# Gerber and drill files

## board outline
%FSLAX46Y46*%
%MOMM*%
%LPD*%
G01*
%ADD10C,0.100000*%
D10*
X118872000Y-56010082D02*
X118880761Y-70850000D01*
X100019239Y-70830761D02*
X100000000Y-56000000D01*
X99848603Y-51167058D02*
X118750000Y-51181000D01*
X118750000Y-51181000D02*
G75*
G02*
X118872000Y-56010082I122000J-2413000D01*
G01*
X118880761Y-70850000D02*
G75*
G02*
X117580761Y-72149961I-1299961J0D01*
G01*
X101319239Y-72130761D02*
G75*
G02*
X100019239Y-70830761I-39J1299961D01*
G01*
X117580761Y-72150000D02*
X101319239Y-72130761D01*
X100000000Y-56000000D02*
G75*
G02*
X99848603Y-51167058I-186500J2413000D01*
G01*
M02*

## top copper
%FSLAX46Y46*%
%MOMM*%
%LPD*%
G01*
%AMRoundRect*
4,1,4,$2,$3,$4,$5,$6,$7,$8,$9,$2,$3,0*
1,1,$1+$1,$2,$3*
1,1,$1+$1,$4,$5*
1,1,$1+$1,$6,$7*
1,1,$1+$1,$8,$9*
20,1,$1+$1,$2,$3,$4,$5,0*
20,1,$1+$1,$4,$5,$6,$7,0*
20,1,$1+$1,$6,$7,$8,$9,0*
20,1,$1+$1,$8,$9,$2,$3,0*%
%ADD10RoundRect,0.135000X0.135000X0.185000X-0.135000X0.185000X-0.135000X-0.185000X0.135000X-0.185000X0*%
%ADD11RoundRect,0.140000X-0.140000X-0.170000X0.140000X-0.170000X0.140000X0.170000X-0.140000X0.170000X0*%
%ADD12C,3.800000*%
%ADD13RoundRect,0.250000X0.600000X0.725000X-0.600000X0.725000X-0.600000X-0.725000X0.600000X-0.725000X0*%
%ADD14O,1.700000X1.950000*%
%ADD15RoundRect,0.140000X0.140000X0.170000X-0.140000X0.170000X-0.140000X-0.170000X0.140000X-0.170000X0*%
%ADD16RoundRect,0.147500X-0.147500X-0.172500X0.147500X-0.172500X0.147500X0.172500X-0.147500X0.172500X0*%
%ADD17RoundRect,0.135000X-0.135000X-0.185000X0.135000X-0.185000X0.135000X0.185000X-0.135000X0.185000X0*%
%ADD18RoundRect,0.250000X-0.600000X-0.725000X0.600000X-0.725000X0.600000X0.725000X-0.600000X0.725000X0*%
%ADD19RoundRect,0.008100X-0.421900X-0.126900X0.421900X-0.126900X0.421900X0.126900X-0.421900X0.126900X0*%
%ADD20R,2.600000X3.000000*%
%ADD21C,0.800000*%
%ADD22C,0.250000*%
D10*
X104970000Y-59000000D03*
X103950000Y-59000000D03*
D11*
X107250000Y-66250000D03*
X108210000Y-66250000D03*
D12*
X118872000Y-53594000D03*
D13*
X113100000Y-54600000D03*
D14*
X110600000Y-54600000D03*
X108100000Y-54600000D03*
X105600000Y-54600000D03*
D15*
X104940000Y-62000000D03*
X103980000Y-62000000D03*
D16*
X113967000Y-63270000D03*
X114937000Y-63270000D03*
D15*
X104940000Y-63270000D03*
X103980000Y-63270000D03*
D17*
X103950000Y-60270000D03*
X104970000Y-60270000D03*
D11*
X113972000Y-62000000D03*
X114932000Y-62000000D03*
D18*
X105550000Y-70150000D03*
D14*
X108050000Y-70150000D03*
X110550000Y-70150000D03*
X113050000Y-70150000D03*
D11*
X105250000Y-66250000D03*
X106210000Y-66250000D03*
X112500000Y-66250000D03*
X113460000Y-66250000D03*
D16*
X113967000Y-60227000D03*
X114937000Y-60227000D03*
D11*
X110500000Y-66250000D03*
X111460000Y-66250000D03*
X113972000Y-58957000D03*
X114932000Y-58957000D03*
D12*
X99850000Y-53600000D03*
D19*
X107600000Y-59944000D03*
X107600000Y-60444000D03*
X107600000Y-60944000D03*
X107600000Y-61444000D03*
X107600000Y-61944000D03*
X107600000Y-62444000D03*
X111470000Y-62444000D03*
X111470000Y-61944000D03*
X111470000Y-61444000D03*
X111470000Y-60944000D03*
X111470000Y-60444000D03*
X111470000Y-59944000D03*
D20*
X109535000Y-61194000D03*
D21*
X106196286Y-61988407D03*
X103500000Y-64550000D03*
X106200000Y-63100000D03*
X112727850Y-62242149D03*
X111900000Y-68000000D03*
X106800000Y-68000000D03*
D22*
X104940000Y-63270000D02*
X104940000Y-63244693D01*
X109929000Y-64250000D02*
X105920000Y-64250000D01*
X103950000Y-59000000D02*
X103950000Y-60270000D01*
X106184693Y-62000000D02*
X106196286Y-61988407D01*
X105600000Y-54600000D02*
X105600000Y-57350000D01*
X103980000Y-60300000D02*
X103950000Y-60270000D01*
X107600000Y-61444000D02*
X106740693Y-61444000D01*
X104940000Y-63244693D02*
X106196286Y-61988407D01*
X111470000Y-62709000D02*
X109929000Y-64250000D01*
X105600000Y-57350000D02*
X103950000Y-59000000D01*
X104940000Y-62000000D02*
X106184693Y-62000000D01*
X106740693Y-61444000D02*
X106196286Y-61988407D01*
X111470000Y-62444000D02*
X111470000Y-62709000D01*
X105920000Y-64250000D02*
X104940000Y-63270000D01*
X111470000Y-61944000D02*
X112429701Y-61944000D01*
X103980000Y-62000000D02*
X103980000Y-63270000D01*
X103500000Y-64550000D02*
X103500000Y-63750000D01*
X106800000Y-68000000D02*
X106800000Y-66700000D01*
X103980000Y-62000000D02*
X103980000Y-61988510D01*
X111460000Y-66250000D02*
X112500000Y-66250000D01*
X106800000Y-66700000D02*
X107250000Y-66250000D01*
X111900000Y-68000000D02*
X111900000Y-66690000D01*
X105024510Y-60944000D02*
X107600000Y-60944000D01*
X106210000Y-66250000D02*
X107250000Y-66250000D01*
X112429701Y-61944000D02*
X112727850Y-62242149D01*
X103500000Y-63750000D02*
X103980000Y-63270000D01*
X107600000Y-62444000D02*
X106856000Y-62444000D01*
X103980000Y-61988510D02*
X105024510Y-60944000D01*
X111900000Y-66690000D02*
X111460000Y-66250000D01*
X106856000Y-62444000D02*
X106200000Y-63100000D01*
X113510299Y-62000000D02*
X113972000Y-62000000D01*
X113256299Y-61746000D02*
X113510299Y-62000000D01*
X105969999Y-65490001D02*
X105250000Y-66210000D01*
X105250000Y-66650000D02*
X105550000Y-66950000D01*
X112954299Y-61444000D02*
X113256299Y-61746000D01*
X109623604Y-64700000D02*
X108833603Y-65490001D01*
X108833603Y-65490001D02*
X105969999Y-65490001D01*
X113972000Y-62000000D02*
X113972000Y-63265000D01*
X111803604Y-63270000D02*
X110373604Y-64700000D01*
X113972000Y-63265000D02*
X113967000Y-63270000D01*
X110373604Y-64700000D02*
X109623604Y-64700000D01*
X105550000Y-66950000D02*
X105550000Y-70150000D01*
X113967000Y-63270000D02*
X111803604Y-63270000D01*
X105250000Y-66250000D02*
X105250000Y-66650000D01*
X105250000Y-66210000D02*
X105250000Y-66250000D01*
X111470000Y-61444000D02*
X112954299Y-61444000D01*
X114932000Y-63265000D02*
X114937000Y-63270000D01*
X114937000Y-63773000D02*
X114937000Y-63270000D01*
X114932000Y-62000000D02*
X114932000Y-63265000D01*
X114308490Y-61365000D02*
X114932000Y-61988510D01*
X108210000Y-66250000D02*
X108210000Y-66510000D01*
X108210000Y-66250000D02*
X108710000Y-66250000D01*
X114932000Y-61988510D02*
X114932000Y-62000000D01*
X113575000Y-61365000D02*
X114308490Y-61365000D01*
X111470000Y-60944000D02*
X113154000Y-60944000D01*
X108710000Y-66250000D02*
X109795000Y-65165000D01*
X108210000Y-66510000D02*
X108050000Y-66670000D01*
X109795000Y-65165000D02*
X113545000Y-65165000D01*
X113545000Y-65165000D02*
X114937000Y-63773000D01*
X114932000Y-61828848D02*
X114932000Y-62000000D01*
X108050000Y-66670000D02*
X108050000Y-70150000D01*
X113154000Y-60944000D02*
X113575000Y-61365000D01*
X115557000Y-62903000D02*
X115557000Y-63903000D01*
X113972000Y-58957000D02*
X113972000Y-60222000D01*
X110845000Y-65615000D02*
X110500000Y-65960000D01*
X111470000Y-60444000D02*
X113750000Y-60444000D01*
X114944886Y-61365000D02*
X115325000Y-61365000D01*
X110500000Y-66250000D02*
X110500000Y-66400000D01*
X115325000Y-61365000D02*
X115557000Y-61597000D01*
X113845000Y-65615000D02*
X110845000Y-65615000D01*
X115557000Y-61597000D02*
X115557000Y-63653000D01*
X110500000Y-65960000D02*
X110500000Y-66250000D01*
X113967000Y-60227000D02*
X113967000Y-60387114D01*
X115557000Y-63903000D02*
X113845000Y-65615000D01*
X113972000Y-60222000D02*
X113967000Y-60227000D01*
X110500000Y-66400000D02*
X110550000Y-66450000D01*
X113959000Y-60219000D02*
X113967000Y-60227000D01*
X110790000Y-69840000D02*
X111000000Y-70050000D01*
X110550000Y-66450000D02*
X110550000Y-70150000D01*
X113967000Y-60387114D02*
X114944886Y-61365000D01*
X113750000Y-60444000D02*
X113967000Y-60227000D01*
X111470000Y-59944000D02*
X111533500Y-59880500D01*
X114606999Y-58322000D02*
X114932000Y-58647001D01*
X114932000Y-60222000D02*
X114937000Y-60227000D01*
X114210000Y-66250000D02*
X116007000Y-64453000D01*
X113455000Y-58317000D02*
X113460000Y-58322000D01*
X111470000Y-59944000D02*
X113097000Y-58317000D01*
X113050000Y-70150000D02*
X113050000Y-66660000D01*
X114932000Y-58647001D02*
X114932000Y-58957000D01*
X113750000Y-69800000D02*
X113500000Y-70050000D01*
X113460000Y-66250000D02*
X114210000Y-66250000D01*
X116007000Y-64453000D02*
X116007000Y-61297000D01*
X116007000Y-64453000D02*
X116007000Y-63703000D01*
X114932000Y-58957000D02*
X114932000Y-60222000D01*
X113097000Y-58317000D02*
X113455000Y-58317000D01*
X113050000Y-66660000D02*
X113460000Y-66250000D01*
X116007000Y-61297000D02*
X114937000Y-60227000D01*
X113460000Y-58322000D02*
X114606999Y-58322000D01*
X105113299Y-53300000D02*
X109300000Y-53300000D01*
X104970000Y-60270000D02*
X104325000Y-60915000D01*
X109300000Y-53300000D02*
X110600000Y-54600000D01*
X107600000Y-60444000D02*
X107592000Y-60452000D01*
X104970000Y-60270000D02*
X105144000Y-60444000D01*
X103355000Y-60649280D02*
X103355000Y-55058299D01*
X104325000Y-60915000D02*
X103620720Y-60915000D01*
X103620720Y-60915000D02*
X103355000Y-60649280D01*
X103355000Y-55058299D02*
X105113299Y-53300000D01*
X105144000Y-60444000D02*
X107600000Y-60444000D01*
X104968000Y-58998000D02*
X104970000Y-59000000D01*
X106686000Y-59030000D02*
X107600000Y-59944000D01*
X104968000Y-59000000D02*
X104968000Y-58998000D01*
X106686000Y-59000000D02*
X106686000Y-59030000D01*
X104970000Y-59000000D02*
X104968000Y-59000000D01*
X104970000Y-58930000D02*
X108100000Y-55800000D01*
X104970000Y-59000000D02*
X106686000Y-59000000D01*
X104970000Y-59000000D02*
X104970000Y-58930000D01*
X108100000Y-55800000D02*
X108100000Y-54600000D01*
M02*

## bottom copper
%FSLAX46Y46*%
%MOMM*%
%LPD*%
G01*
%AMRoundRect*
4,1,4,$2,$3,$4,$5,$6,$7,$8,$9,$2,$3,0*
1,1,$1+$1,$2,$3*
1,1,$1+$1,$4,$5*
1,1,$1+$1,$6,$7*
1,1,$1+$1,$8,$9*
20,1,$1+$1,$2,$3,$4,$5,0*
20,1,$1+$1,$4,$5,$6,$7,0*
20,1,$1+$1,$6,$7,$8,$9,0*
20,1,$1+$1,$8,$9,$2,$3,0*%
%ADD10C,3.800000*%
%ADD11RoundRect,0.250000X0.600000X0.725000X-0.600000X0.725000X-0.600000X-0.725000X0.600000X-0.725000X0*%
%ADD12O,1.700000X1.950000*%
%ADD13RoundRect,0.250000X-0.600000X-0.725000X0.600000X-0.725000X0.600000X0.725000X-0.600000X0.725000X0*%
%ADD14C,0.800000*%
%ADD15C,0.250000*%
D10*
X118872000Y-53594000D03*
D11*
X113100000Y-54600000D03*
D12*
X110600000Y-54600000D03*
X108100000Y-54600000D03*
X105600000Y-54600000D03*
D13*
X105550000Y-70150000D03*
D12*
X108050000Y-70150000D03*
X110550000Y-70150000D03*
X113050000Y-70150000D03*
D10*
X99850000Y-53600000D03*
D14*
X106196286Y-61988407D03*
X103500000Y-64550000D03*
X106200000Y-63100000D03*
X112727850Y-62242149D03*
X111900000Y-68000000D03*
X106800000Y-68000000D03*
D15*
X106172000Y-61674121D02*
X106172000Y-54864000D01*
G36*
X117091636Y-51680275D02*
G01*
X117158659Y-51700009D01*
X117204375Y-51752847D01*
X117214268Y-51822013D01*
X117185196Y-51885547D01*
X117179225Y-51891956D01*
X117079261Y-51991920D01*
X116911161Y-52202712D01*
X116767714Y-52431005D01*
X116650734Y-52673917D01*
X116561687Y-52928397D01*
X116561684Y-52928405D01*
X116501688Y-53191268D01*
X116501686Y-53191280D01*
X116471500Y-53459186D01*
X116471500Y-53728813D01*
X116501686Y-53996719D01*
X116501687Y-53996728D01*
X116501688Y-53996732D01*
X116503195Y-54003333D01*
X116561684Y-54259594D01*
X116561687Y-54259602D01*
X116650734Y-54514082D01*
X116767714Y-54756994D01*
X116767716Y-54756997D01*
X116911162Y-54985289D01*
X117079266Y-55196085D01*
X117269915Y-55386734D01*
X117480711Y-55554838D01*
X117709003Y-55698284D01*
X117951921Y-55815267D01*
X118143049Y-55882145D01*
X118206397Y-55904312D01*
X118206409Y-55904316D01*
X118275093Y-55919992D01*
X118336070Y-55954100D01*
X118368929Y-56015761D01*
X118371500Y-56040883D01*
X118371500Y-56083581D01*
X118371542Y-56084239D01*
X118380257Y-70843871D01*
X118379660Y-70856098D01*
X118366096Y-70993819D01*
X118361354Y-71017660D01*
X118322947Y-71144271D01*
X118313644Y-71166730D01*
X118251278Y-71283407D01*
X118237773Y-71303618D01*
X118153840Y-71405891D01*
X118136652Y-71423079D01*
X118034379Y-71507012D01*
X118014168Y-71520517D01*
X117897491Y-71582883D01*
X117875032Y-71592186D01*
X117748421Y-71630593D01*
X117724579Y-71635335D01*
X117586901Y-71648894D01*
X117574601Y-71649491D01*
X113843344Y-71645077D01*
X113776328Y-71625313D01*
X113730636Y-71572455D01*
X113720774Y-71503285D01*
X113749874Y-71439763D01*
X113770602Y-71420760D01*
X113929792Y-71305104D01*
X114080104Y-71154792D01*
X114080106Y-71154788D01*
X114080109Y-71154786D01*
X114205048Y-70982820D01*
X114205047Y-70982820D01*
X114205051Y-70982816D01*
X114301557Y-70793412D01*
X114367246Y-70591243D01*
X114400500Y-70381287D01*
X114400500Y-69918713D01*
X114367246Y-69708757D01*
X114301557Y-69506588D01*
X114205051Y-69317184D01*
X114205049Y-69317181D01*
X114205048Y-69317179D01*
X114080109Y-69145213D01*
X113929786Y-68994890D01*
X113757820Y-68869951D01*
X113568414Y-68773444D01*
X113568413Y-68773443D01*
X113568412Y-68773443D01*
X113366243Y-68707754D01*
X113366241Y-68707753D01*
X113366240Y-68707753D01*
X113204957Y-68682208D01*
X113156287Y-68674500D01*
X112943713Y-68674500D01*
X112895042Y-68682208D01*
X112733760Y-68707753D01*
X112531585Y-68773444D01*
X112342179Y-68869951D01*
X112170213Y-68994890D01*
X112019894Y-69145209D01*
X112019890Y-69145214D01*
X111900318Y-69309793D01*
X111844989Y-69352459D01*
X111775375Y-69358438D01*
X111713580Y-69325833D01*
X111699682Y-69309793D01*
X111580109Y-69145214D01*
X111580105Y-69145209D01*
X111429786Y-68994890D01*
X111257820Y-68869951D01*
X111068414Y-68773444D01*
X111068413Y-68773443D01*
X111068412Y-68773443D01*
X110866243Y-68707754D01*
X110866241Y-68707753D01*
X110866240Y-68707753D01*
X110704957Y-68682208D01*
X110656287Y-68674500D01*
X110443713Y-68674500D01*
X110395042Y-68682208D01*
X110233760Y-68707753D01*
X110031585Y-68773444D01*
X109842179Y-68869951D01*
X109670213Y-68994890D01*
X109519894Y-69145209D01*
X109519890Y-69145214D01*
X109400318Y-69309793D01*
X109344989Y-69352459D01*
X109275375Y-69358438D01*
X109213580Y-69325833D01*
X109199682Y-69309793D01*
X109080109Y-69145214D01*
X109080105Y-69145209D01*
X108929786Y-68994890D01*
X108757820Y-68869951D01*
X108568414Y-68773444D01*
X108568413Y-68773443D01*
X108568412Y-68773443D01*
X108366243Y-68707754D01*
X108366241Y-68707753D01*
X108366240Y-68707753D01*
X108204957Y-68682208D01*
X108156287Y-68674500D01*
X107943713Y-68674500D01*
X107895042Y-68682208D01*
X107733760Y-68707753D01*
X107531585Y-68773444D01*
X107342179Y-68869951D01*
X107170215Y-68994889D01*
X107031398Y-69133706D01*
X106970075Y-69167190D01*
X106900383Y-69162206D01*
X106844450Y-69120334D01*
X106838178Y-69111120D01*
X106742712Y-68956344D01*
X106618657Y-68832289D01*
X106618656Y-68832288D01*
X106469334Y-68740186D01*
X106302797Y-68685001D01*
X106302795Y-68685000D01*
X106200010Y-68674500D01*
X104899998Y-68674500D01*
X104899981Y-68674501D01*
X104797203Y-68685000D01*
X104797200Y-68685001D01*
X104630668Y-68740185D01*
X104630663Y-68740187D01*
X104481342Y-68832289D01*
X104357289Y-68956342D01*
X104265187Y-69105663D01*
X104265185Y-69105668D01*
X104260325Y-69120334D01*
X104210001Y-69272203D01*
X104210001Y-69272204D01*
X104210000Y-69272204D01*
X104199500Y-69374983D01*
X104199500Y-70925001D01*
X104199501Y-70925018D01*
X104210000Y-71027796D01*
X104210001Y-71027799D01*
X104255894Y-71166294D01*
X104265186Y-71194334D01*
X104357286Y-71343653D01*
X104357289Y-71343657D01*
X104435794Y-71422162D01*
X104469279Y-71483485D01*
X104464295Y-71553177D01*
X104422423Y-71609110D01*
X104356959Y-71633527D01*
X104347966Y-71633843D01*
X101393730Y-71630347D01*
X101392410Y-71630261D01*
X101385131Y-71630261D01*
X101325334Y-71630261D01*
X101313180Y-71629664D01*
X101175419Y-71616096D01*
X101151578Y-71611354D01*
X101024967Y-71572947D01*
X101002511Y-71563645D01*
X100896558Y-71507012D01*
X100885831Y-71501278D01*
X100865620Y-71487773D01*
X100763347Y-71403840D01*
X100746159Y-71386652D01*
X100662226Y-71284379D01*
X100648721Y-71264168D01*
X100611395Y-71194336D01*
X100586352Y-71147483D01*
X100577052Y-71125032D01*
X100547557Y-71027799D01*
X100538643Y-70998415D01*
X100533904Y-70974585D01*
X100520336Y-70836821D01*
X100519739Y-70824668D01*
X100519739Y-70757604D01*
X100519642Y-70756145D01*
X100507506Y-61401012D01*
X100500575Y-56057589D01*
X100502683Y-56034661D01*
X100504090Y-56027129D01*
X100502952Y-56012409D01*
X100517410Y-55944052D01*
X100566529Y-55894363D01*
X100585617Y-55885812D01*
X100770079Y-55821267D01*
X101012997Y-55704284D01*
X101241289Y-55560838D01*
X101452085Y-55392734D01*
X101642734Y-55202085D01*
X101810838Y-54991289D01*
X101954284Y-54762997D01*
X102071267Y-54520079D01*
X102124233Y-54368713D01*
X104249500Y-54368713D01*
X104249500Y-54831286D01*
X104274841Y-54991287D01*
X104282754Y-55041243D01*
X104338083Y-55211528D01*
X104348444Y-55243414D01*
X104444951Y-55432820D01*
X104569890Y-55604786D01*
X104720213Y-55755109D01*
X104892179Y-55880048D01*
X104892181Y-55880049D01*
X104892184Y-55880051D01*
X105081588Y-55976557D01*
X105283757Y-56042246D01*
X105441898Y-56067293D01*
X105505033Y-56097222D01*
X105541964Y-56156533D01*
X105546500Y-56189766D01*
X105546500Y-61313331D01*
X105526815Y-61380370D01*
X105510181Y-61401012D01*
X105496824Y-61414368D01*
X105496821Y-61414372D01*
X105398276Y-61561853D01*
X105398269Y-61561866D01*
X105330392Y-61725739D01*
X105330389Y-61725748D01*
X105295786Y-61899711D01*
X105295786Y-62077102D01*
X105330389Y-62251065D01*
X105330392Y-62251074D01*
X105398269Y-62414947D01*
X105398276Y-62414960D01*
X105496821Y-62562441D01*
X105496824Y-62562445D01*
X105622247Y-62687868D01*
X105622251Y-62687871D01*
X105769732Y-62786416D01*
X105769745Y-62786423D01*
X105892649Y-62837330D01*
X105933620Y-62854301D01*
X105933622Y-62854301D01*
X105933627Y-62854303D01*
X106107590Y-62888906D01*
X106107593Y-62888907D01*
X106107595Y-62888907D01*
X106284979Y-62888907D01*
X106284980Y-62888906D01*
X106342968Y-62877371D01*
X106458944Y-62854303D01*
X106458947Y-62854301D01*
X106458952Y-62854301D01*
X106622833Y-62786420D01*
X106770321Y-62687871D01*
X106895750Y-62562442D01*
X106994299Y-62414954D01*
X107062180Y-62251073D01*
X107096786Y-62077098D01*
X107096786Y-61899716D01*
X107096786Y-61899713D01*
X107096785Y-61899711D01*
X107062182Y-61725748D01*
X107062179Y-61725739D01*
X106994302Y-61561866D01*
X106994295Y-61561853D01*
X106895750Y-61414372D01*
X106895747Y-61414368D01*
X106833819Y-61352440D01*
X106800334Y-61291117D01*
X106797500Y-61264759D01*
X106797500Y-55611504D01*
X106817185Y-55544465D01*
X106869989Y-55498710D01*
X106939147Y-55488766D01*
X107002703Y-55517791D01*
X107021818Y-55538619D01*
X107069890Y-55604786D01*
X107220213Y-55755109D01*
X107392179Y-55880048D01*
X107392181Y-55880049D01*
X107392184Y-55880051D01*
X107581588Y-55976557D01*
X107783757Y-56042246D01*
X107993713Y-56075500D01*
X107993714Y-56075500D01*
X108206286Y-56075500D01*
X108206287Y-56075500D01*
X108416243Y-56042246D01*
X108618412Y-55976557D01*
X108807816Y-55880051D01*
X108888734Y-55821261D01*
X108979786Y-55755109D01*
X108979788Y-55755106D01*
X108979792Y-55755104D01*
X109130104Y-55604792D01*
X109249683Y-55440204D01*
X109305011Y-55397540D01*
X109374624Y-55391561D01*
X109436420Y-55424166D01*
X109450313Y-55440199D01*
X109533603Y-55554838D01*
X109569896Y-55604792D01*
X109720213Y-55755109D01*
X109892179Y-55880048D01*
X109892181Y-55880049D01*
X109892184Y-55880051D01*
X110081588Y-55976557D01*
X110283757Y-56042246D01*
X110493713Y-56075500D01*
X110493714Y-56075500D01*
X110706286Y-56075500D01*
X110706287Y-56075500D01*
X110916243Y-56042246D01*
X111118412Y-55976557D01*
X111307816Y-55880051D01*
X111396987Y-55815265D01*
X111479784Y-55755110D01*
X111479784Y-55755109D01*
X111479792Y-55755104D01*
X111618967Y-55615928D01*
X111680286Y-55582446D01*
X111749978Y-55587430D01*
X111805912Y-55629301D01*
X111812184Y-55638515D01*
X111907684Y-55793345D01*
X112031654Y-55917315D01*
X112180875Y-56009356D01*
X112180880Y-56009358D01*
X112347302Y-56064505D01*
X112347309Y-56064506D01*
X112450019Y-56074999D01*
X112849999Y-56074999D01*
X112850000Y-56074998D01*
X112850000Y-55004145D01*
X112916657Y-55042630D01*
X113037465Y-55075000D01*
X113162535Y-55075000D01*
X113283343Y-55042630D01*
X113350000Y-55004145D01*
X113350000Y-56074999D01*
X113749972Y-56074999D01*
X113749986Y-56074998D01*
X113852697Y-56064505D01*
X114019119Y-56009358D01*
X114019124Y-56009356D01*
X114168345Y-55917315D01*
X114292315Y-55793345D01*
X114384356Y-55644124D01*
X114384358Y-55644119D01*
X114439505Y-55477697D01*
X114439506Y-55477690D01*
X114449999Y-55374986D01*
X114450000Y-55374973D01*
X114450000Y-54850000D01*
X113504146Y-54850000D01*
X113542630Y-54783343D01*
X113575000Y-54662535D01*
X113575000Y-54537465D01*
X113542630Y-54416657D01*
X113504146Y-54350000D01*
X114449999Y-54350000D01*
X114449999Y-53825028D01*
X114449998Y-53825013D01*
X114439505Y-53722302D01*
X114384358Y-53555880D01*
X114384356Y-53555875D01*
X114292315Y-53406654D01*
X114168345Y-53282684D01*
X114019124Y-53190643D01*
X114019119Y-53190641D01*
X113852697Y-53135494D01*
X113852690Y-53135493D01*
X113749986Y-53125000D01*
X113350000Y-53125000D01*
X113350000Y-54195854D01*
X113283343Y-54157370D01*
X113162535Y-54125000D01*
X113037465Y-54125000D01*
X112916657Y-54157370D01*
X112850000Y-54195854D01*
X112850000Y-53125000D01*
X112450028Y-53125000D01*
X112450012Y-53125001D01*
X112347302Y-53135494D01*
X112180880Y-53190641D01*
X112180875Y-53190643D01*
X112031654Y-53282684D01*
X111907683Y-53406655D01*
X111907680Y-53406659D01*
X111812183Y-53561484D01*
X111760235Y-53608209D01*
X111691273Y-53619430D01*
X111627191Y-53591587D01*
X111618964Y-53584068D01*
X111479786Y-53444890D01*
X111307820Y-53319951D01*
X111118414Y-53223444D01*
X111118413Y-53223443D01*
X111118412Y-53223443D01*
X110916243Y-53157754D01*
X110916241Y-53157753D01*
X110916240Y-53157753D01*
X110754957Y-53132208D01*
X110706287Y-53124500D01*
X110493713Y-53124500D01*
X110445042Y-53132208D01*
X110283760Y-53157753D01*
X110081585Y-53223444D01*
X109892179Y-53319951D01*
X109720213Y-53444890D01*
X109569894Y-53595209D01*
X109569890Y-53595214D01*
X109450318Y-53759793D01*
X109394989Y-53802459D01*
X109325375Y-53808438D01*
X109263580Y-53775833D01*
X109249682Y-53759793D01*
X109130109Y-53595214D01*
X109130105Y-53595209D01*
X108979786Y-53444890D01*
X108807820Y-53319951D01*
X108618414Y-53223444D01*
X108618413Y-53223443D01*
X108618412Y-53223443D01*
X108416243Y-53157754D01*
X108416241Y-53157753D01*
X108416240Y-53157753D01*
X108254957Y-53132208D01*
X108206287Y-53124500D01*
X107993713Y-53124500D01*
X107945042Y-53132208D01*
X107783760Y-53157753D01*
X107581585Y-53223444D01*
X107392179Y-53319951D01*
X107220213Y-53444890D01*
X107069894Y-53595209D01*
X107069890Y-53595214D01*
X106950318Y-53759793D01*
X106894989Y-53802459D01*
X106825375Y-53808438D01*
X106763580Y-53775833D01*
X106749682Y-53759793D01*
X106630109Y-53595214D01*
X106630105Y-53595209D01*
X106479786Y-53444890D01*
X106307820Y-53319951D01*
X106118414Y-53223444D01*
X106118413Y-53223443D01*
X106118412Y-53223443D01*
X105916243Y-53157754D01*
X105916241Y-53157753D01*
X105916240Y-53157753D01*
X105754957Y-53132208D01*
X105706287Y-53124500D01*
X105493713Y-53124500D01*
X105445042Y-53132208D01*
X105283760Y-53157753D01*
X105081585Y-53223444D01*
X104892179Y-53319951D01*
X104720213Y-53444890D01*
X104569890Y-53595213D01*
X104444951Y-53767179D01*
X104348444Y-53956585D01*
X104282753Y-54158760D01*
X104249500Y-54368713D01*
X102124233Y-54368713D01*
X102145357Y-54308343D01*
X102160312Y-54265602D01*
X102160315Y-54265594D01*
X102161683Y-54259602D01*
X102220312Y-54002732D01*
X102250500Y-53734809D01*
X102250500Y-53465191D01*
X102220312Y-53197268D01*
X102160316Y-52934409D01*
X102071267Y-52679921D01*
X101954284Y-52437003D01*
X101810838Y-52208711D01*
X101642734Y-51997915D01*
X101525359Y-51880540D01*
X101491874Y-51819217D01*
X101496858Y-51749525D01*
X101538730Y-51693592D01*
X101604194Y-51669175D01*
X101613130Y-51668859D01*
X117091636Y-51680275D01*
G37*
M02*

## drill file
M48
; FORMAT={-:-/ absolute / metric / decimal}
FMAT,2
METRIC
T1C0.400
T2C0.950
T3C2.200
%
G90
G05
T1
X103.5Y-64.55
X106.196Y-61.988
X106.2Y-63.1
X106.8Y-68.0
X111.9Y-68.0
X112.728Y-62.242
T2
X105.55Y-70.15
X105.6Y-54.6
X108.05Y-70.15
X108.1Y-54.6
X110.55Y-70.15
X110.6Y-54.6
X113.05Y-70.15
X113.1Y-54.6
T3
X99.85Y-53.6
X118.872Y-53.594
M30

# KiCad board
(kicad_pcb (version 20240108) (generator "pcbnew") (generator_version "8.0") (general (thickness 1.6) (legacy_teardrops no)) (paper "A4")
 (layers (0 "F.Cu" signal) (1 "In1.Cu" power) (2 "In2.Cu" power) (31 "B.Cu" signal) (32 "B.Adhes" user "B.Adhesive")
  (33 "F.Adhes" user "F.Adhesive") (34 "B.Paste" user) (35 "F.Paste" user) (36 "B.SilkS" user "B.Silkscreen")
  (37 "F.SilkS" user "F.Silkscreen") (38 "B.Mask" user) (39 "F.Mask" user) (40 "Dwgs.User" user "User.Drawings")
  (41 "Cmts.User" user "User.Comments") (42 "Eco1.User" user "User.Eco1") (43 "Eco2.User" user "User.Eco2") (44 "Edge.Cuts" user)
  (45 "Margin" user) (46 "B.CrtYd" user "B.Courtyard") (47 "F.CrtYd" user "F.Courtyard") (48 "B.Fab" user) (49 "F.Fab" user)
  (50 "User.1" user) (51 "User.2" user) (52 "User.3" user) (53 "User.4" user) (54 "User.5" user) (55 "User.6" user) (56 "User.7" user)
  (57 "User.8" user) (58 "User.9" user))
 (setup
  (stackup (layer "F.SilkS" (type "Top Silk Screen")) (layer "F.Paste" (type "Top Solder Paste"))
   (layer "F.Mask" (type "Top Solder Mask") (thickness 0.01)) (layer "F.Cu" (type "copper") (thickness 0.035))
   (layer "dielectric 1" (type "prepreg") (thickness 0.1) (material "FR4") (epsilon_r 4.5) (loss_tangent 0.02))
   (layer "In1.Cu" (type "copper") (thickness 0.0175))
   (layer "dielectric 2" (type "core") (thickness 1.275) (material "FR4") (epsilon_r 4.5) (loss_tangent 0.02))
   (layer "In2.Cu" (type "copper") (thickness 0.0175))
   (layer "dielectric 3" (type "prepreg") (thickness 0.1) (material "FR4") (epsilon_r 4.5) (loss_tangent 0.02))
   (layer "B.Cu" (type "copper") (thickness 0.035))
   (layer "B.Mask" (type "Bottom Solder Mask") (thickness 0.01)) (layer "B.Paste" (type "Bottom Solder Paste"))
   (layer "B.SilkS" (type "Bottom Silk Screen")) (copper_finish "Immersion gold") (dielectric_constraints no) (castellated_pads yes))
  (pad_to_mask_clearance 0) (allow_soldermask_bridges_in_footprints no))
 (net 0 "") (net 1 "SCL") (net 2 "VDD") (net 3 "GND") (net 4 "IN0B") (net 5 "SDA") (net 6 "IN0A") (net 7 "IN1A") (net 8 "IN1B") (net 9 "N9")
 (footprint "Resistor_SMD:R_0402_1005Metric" (layer "F.Cu") (at 104.46 59 180)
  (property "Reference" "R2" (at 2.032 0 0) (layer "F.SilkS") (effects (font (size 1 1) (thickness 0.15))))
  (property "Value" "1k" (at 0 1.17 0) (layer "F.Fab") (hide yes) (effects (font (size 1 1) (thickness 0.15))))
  (pad "1" smd roundrect (at -0.51 0 180) (size 0.54 0.64) (layers "F.Cu" "F.Paste" "F.Mask") (roundrect_rratio 0.25) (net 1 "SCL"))
  (pad "2" smd roundrect (at 0.51 0 180) (size 0.54 0.64) (layers "F.Cu" "F.Paste" "F.Mask") (roundrect_rratio 0.25) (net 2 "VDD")))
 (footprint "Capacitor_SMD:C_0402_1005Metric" (layer "F.Cu") (at 107.73 66.25)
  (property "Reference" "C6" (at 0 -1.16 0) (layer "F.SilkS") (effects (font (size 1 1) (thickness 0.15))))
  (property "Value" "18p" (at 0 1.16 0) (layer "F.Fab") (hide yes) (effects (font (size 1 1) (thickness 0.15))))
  (pad "1" smd roundrect (at -0.48 0) (size 0.56 0.62) (layers "F.Cu" "F.Paste" "F.Mask") (roundrect_rratio 0.25) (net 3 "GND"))
  (pad "2" smd roundrect (at 0.48 0) (size 0.56 0.62) (layers "F.Cu" "F.Paste" "F.Mask") (roundrect_rratio 0.25) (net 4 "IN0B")))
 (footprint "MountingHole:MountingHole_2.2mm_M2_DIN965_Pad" (layer "F.Cu") (at 118.872 53.594)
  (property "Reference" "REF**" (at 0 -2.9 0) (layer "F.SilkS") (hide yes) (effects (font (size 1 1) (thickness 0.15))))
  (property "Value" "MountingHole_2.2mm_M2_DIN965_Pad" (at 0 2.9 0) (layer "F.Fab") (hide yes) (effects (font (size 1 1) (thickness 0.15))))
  (pad "1" thru_hole circle (at 0 0) (size 3.8 3.8) (drill 2.2) (layers "*.Cu" "*.Mask") (remove_unused_layers no)))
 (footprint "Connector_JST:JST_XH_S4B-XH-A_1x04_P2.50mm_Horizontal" (layer "F.Cu") (at 113.1 54.6 180)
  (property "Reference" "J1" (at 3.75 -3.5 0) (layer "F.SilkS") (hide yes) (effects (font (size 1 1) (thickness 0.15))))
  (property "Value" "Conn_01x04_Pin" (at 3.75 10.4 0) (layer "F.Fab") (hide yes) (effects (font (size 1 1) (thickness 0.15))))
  (pad "1" thru_hole roundrect (at 0 0 180) (size 1.7 1.95) (drill 0.95) (layers "*.Cu" "*.Mask") (remove_unused_layers no)
   (roundrect_rratio 0.147059) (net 3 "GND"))
  (pad "2" thru_hole oval (at 2.5 0 180) (size 1.7 1.95) (drill 0.95) (layers "*.Cu" "*.Mask") (remove_unused_layers no) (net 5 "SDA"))
  (pad "3" thru_hole oval (at 5 0 180) (size 1.7 1.95) (drill 0.95) (layers "*.Cu" "*.Mask") (remove_unused_layers no) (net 1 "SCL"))
  (pad "4" thru_hole oval (at 7.5 0 180) (size 1.7 1.95) (drill 0.95) (layers "*.Cu" "*.Mask") (remove_unused_layers no) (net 2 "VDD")))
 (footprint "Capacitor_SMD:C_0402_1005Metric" (layer "F.Cu") (at 104.46 62 180)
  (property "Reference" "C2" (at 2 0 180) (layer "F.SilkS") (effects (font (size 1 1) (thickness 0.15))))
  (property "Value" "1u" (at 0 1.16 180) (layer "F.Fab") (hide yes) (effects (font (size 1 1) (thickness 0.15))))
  (pad "1" smd roundrect (at -0.48 0 180) (size 0.56 0.62) (layers "F.Cu" "F.Paste" "F.Mask") (roundrect_rratio 0.25) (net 2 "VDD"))
  (pad "2" smd roundrect (at 0.48 0 180) (size 0.56 0.62) (layers "F.Cu" "F.Paste" "F.Mask") (roundrect_rratio 0.25) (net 3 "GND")))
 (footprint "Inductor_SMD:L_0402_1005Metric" (layer "F.Cu") (at 114.452 63.27)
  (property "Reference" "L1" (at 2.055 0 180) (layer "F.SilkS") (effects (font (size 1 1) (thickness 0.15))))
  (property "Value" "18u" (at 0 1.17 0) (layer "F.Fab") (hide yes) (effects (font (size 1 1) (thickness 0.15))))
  (pad "1" smd roundrect (at -0.485 0) (size 0.59 0.64) (layers "F.Cu" "F.Paste" "F.Mask") (roundrect_rratio 0.25) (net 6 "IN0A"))
  (pad "2" smd roundrect (at 0.485 0) (size 0.59 0.64) (layers "F.Cu" "F.Paste" "F.Mask") (roundrect_rratio 0.25) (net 4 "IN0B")))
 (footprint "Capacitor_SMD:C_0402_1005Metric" (layer "F.Cu") (at 104.46 63.27 180)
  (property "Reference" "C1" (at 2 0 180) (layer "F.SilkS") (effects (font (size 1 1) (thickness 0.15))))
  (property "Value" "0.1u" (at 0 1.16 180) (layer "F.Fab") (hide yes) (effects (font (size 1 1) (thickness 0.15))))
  (pad "1" smd roundrect (at -0.48 0 180) (size 0.56 0.62) (layers "F.Cu" "F.Paste" "F.Mask") (roundrect_rratio 0.25) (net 2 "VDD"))
  (pad "2" smd roundrect (at 0.48 0 180) (size 0.56 0.62) (layers "F.Cu" "F.Paste" "F.Mask") (roundrect_rratio 0.25) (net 3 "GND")))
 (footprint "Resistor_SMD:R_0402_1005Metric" (layer "F.Cu") (at 104.46 60.27)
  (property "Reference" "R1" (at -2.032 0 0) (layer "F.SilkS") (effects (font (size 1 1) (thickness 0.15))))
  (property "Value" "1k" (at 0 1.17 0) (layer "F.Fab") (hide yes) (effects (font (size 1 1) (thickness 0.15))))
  (pad "1" smd roundrect (at -0.51 0) (size 0.54 0.64) (layers "F.Cu" "F.Paste" "F.Mask") (roundrect_rratio 0.25) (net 2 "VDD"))
  (pad "2" smd roundrect (at 0.51 0) (size 0.54 0.64) (layers "F.Cu" "F.Paste" "F.Mask") (roundrect_rratio 0.25) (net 5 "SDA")))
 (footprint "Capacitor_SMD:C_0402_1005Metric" (layer "F.Cu") (at 114.452 62)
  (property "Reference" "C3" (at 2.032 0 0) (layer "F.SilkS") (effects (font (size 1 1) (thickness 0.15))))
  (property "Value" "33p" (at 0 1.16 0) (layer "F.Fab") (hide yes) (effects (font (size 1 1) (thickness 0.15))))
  (pad "1" smd roundrect (at -0.48 0) (size 0.56 0.62) (layers "F.Cu" "F.Paste" "F.Mask") (roundrect_rratio 0.25) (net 6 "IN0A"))
  (pad "2" smd roundrect (at 0.48 0) (size 0.56 0.62) (layers "F.Cu" "F.Paste" "F.Mask") (roundrect_rratio 0.25) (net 4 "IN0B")))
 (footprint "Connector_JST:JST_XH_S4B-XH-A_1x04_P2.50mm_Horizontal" (layer "F.Cu") (at 105.55 70.15)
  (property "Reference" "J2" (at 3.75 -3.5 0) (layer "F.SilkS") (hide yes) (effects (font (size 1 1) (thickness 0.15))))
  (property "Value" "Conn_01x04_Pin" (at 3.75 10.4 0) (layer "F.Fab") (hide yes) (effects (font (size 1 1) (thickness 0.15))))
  (pad "1" thru_hole roundrect (at 0 0) (size 1.7 1.95) (drill 0.95) (layers "*.Cu" "*.Mask") (remove_unused_layers no)
   (roundrect_rratio 0.147059) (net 6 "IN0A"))
  (pad "2" thru_hole oval (at 2.5 0) (size 1.7 1.95) (drill 0.95) (layers "*.Cu" "*.Mask") (remove_unused_layers no) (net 4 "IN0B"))
  (pad "3" thru_hole oval (at 5 0) (size 1.7 1.95) (drill 0.95) (layers "*.Cu" "*.Mask") (remove_unused_layers no) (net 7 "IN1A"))
  (pad "4" thru_hole oval (at 7.5 0) (size 1.7 1.95) (drill 0.95) (layers "*.Cu" "*.Mask") (remove_unused_layers no) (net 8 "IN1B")))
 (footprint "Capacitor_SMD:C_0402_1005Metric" (layer "F.Cu") (at 105.73 66.25)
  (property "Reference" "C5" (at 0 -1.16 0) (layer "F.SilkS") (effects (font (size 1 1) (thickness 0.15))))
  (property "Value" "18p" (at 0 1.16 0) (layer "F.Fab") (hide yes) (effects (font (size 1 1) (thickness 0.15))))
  (pad "1" smd roundrect (at -0.48 0) (size 0.56 0.62) (layers "F.Cu" "F.Paste" "F.Mask") (roundrect_rratio 0.25) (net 6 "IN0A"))
  (pad "2" smd roundrect (at 0.48 0) (size 0.56 0.62) (layers "F.Cu" "F.Paste" "F.Mask") (roundrect_rratio 0.25) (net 3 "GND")))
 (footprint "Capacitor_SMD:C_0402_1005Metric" (layer "F.Cu") (at 112.98 66.25)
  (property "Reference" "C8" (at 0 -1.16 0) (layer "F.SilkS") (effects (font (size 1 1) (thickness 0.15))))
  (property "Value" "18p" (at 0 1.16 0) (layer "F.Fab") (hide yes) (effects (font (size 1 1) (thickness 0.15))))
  (pad "1" smd roundrect (at -0.48 0) (size 0.56 0.62) (layers "F.Cu" "F.Paste" "F.Mask") (roundrect_rratio 0.25) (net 3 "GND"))
  (pad "2" smd roundrect (at 0.48 0) (size 0.56 0.62) (layers "F.Cu" "F.Paste" "F.Mask") (roundrect_rratio 0.25) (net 8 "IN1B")))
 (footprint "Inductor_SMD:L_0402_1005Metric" (layer "F.Cu") (at 114.452 60.227)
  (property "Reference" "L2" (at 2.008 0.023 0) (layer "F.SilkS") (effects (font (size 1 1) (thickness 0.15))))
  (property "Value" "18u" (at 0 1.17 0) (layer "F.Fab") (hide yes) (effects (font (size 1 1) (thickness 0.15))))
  (pad "1" smd roundrect (at -0.485 0) (size 0.59 0.64) (layers "F.Cu" "F.Paste" "F.Mask") (roundrect_rratio 0.25) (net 7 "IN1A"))
  (pad "2" smd roundrect (at 0.485 0) (size 0.59 0.64) (layers "F.Cu" "F.Paste" "F.Mask") (roundrect_rratio 0.25) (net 8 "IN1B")))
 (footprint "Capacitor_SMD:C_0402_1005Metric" (layer "F.Cu") (at 110.98 66.25)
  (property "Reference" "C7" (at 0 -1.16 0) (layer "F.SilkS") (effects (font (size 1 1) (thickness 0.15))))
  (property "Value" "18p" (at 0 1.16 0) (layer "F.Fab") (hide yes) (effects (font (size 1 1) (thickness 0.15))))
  (pad "1" smd roundrect (at -0.48 0) (size 0.56 0.62) (layers "F.Cu" "F.Paste" "F.Mask") (roundrect_rratio 0.25) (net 7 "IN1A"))
  (pad "2" smd roundrect (at 0.48 0) (size 0.56 0.62) (layers "F.Cu" "F.Paste" "F.Mask") (roundrect_rratio 0.25) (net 3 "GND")))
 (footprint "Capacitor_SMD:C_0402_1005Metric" (layer "F.Cu") (at 114.452 58.957)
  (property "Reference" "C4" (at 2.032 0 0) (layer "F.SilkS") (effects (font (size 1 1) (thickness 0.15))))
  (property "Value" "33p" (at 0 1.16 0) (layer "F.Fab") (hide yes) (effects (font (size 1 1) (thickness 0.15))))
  (pad "1" smd roundrect (at -0.48 0) (size 0.56 0.62) (layers "F.Cu" "F.Paste" "F.Mask") (roundrect_rratio 0.25) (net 7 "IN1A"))
  (pad "2" smd roundrect (at 0.48 0) (size 0.56 0.62) (layers "F.Cu" "F.Paste" "F.Mask") (roundrect_rratio 0.25) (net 8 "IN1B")))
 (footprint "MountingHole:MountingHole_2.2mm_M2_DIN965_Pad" (layer "F.Cu") (at 99.85 53.6)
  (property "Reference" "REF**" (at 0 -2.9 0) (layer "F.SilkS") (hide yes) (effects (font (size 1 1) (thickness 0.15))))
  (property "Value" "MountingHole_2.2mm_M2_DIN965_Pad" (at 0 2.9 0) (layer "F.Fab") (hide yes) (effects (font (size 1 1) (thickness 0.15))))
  (pad "1" thru_hole circle (at 0 0) (size 3.8 3.8) (drill 2.2) (layers "*.Cu" "*.Mask") (remove_unused_layers no)))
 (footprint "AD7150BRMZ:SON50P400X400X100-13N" (layer "F.Cu") (at 109.535 61.194)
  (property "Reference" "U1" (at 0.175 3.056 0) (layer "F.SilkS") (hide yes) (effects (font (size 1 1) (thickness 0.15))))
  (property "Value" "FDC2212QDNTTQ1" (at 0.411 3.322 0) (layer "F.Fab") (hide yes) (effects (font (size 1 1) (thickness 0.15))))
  (pad "1" smd roundrect (at -1.935 -1.25) (size 0.86 0.27) (layers "F.Cu" "F.Paste" "F.Mask") (roundrect_rratio 0.03) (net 1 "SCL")
   (solder_mask_margin 0.102))
  (pad "2" smd roundrect (at -1.935 -0.75) (size 0.86 0.27) (layers "F.Cu" "F.Paste" "F.Mask") (roundrect_rratio 0.03) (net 5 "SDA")
   (solder_mask_margin 0.102))
  (pad "3" smd roundrect (at -1.935 -0.25) (size 0.86 0.27) (layers "F.Cu" "F.Paste" "F.Mask") (roundrect_rratio 0.03) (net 3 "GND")
   (solder_mask_margin 0.102))
  (pad "4" smd roundrect (at -1.935 0.25) (size 0.86 0.27) (layers "F.Cu" "F.Paste" "F.Mask") (roundrect_rratio 0.03) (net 2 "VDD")
   (solder_mask_margin 0.102))
  (pad "5" smd roundrect (at -1.935 0.75) (size 0.86 0.27) (layers "F.Cu" "F.Paste" "F.Mask") (roundrect_rratio 0.03) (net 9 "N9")
   (solder_mask_margin 0.102))
  (pad "6" smd roundrect (at -1.935 1.25) (size 0.86 0.27) (layers "F.Cu" "F.Paste" "F.Mask") (roundrect_rratio 0.03) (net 3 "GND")
   (solder_mask_margin 0.102))
  (pad "7" smd roundrect (at 1.935 1.25) (size 0.86 0.27) (layers "F.Cu" "F.Paste" "F.Mask") (roundrect_rratio 0.03) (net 2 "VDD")
   (solder_mask_margin 0.102))
  (pad "8" smd roundrect (at 1.935 0.75) (size 0.86 0.27) (layers "F.Cu" "F.Paste" "F.Mask") (roundrect_rratio 0.03) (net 3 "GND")
   (solder_mask_margin 0.102))
  (pad "9" smd roundrect (at 1.935 0.25) (size 0.86 0.27) (layers "F.Cu" "F.Paste" "F.Mask") (roundrect_rratio 0.03) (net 6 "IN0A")
   (solder_mask_margin 0.102))
  (pad "10" smd roundrect (at 1.935 -0.25) (size 0.86 0.27) (layers "F.Cu" "F.Paste" "F.Mask") (roundrect_rratio 0.03) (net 4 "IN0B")
   (solder_mask_margin 0.102))
  (pad "11" smd roundrect (at 1.935 -0.75) (size 0.86 0.27) (layers "F.Cu" "F.Paste" "F.Mask") (roundrect_rratio 0.03) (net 7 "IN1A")
   (solder_mask_margin 0.102))
  (pad "12" smd roundrect (at 1.935 -1.25) (size 0.86 0.27) (layers "F.Cu" "F.Paste" "F.Mask") (roundrect_rratio 0.03) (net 8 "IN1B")
   (solder_mask_margin 0.102))
  (pad "13" smd rect (at 0 0) (size 2.6 3) (layers "F.Cu" "F.Mask") (solder_mask_margin 0.102)))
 (gr_line (start 118.872 56.010082) (end 118.880761 70.85) (stroke (width 0.1) (type default)) (layer "Edge.Cuts"))
 (gr_line (start 100.019239 70.830761) (end 100 56) (stroke (width 0.1) (type default)) (layer "Edge.Cuts"))
 (gr_line (start 99.848603 51.167058) (end 118.75 51.181) (stroke (width 0.1) (type default)) (layer "Edge.Cuts"))
 (gr_arc (start 118.75 51.181) (mid 121.287311 53.532981) (end 118.872 56.010082) (stroke (width 0.1) (type default)) (layer "Edge.Cuts"))
 (gr_arc (start 118.880761 70.85) (mid 118.5 71.769239) (end 117.580761 72.15) (stroke (width 0.1) (type default)) (layer "Edge.Cuts"))
 (gr_arc (start 101.319239 72.130761) (mid 100.4 71.75) (end 100.019239 70.830761) (stroke (width 0.1) (type default)) (layer "Edge.Cuts"))
 (gr_line (start 117.580761 72.15) (end 101.319239 72.130761) (stroke (width 0.1) (type default)) (layer "Edge.Cuts"))
 (gr_arc (start 100 56) (mid 97.394497 53.662778) (end 99.848603 51.167058) (stroke (width 0.1) (type default)) (layer "Edge.Cuts"))
 (segment (start 104.94 63.27) (end 104.94 63.244693) (width 0.25) (layer "F.Cu") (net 2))
 (segment (start 109.929 64.25) (end 105.92 64.25) (width 0.25) (layer "F.Cu") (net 2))
 (segment (start 103.95 59) (end 103.95 60.27) (width 0.25) (layer "F.Cu") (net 2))
 (segment (start 106.184693 62) (end 106.196286 61.988407) (width 0.25) (layer "F.Cu") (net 2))
 (segment (start 105.6 54.6) (end 105.6 57.35) (width 0.25) (layer "F.Cu") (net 2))
 (segment (start 103.98 60.3) (end 103.95 60.27) (width 0.25) (layer "F.Cu") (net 2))
 (segment (start 107.6 61.444) (end 106.740693 61.444) (width 0.25) (layer "F.Cu") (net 2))
 (segment (start 104.94 63.244693) (end 106.196286 61.988407) (width 0.25) (layer "F.Cu") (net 2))
 (segment (start 111.47 62.709) (end 109.929 64.25) (width 0.25) (layer "F.Cu") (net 2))
 (segment (start 105.6 57.35) (end 103.95 59) (width 0.25) (layer "F.Cu") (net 2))
 (segment (start 104.94 62) (end 106.184693 62) (width 0.25) (layer "F.Cu") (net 2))
 (segment (start 106.740693 61.444) (end 106.196286 61.988407) (width 0.25) (layer "F.Cu") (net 2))
 (segment (start 111.47 62.444) (end 111.47 62.709) (width 0.25) (layer "F.Cu") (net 2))
 (segment (start 105.92 64.25) (end 104.94 63.27) (width 0.25) (layer "F.Cu") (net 2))
 (via (at 106.196286 61.988407) (size 0.8) (drill 0.4) (layers "F.Cu" "B.Cu") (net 2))
 (segment (start 106.172 61.674121) (end 106.172 54.864) (width 0.25) (layer "B.Cu") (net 2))
 (segment (start 111.47 61.944) (end 112.429701 61.944) (width 0.25) (layer "F.Cu") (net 3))
 (segment (start 103.98 62) (end 103.98 63.27) (width 0.25) (layer "F.Cu") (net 3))
 (segment (start 103.5 64.55) (end 103.5 63.75) (width 0.25) (layer "F.Cu") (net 3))
 (segment (start 106.8 68) (end 106.8 66.7) (width 0.25) (layer "F.Cu") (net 3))
 (segment (start 103.98 62) (end 103.98 61.98851) (width 0.25) (layer "F.Cu") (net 3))
 (segment (start 111.46 66.25) (end 112.5 66.25) (width 0.25) (layer "F.Cu") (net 3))
 (segment (start 106.8 66.7) (end 107.25 66.25) (width 0.25) (layer "F.Cu") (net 3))
 (segment (start 111.9 68) (end 111.9 66.69) (width 0.25) (layer "F.Cu") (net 3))
 (segment (start 105.02451 60.944) (end 107.6 60.944) (width 0.25) (layer "F.Cu") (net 3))
 (segment (start 106.21 66.25) (end 107.25 66.25) (width 0.25) (layer "F.Cu") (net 3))
 (segment (start 112.429701 61.944) (end 112.72785 62.242149) (width 0.25) (layer "F.Cu") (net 3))
 (segment (start 103.5 63.75) (end 103.98 63.27) (width 0.25) (layer "F.Cu") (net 3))
 (segment (start 107.6 62.444) (end 106.856 62.444) (width 0.25) (layer "F.Cu") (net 3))
 (segment (start 103.98 61.98851) (end 105.02451 60.944) (width 0.25) (layer "F.Cu") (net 3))
 (segment (start 111.9 66.69) (end 111.46 66.25) (width 0.25) (layer "F.Cu") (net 3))
 (segment (start 106.856 62.444) (end 106.2 63.1) (width 0.25) (layer "F.Cu") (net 3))
 (via (at 103.5 64.55) (size 0.8) (drill 0.4) (layers "F.Cu" "B.Cu") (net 3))
 (via (at 106.2 63.1) (size 0.8) (drill 0.4) (layers "F.Cu" "B.Cu") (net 3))
 (via (at 112.72785 62.242149) (size 0.8) (drill 0.4) (layers "F.Cu" "B.Cu") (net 3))
 (via (at 111.9 68) (size 0.8) (drill 0.4) (layers "F.Cu" "B.Cu") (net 3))
 (via (at 106.8 68) (size 0.8) (drill 0.4) (layers "F.Cu" "B.Cu") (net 3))
 (segment (start 113.510299 62) (end 113.972 62) (width 0.25) (layer "F.Cu") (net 6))
 (segment (start 113.256299 61.746) (end 113.510299 62) (width 0.25) (layer "F.Cu") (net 6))
 (segment (start 105.969999 65.490001) (end 105.25 66.21) (width 0.25) (layer "F.Cu") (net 6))
 (segment (start 105.25 66.65) (end 105.55 66.95) (width 0.25) (layer "F.Cu") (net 6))
 (segment (start 112.954299 61.444) (end 113.256299 61.746) (width 0.25) (layer "F.Cu") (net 6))
 (segment (start 109.623604 64.7) (end 108.833603 65.490001) (width 0.25) (layer "F.Cu") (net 6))
 (segment (start 108.833603 65.490001) (end 105.969999 65.490001) (width 0.25) (layer "F.Cu") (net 6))
 (segment (start 113.972 62) (end 113.972 63.265) (width 0.25) (layer "F.Cu") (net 6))
 (segment (start 111.803604 63.27) (end 110.373604 64.7) (width 0.25) (layer "F.Cu") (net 6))
 (segment (start 113.972 63.265) (end 113.967 63.27) (width 0.25) (layer "F.Cu") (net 6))
 (segment (start 110.373604 64.7) (end 109.623604 64.7) (width 0.25) (layer "F.Cu") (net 6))
 (segment (start 105.55 66.95) (end 105.55 70.15) (width 0.25) (layer "F.Cu") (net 6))
 (segment (start 113.967 63.27) (end 111.803604 63.27) (width 0.25) (layer "F.Cu") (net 6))
 (segment (start 105.25 66.25) (end 105.25 66.65) (width 0.25) (layer "F.Cu") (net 6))
 (segment (start 105.25 66.21) (end 105.25 66.25) (width 0.25) (layer "F.Cu") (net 6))
 (segment (start 111.47 61.444) (end 112.954299 61.444) (width 0.25) (layer "F.Cu") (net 6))
 (segment (start 114.932 63.265) (end 114.937 63.27) (width 0.25) (layer "F.Cu") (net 4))
 (segment (start 114.937 63.773) (end 114.937 63.27) (width 0.25) (layer "F.Cu") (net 4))
 (segment (start 114.932 62) (end 114.932 63.265) (width 0.25) (layer "F.Cu") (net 4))
 (segment (start 114.30849 61.365) (end 114.932 61.98851) (width 0.25) (layer "F.Cu") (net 4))
 (segment (start 108.21 66.25) (end 108.21 66.51) (width 0.25) (layer "F.Cu") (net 4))
 (segment (start 108.21 66.25) (end 108.71 66.25) (width 0.25) (layer "F.Cu") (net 4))
 (segment (start 114.932 61.98851) (end 114.932 62) (width 0.25) (layer "F.Cu") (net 4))
 (segment (start 113.575 61.365) (end 114.30849 61.365) (width 0.25) (layer "F.Cu") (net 4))
 (segment (start 111.47 60.944) (end 113.154 60.944) (width 0.25) (layer "F.Cu") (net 4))
 (segment (start 108.71 66.25) (end 109.795 65.165) (width 0.25) (layer "F.Cu") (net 4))
 (segment (start 108.21 66.51) (end 108.05 66.67) (width 0.25) (layer "F.Cu") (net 4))
 (segment (start 109.795 65.165) (end 113.545 65.165) (width 0.25) (layer "F.Cu") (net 4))
 (segment (start 113.545 65.165) (end 114.937 63.773) (width 0.25) (layer "F.Cu") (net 4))
 (segment (start 114.932 61.828848) (end 114.932 62) (width 0.25) (layer "F.Cu") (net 4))
 (segment (start 108.05 66.67) (end 108.05 70.15) (width 0.25) (layer "F.Cu") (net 4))
 (segment (start 113.154 60.944) (end 113.575 61.365) (width 0.25) (layer "F.Cu") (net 4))
 (segment (start 115.557 62.903) (end 115.557 63.903) (width 0.25) (layer "F.Cu") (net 7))
 (segment (start 113.972 58.957) (end 113.972 60.222) (width 0.25) (layer "F.Cu") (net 7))
 (segment (start 110.845 65.615) (end 110.5 65.96) (width 0.25) (layer "F.Cu") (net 7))
 (segment (start 111.47 60.444) (end 113.75 60.444) (width 0.25) (layer "F.Cu") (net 7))
 (segment (start 114.944886 61.365) (end 115.325 61.365) (width 0.25) (layer "F.Cu") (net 7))
 (segment (start 110.5 66.25) (end 110.5 66.4) (width 0.25) (layer "F.Cu") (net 7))
 (segment (start 115.325 61.365) (end 115.557 61.597) (width 0.25) (layer "F.Cu") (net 7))
 (segment (start 113.845 65.615) (end 110.845 65.615) (width 0.25) (layer "F.Cu") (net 7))
 (segment (start 115.557 61.597) (end 115.557 63.653) (width 0.25) (layer "F.Cu") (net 7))
 (segment (start 110.5 65.96) (end 110.5 66.25) (width 0.25) (layer "F.Cu") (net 7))
 (segment (start 113.967 60.227) (end 113.967 60.387114) (width 0.25) (layer "F.Cu") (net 7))
 (segment (start 115.557 63.903) (end 113.845 65.615) (width 0.25) (layer "F.Cu") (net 7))
 (segment (start 113.972 60.222) (end 113.967 60.227) (width 0.25) (layer "F.Cu") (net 7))
 (segment (start 110.5 66.4) (end 110.55 66.45) (width 0.25) (layer "F.Cu") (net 7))
 (segment (start 113.959 60.219) (end 113.967 60.227) (width 0.25) (layer "F.Cu") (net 7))
 (segment (start 110.79 69.84) (end 111 70.05) (width 0.25) (layer "F.Cu") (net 7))
 (segment (start 110.55 66.45) (end 110.55 70.15) (width 0.25) (layer "F.Cu") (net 7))
 (segment (start 113.967 60.387114) (end 114.944886 61.365) (width 0.25) (layer "F.Cu") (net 7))
 (segment (start 113.75 60.444) (end 113.967 60.227) (width 0.25) (layer "F.Cu") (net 7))
 (segment (start 111.47 59.944) (end 111.5335 59.8805) (width 0.25) (layer "F.Cu") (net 8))
 (segment (start 114.606999 58.322) (end 114.932 58.647001) (width 0.25) (layer "F.Cu") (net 8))
 (segment (start 114.932 60.222) (end 114.937 60.227) (width 0.25) (layer "F.Cu") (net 8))
 (segment (start 114.21 66.25) (end 116.007 64.453) (width 0.25) (layer "F.Cu") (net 8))
 (segment (start 113.455 58.317) (end 113.46 58.322) (width 0.25) (layer "F.Cu") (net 8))
 (segment (start 111.47 59.944) (end 113.097 58.317) (width 0.25) (layer "F.Cu") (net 8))
 (segment (start 113.05 70.15) (end 113.05 66.66) (width 0.25) (layer "F.Cu") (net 8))
 (segment (start 114.932 58.647001) (end 114.932 58.957) (width 0.25) (layer "F.Cu") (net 8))
 (segment (start 113.75 69.8) (end 113.5 70.05) (width 0.25) (layer "F.Cu") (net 8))
 (segment (start 113.46 66.25) (end 114.21 66.25) (width 0.25) (layer "F.Cu") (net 8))
 (segment (start 116.007 64.453) (end 116.007 61.297) (width 0.25) (layer "F.Cu") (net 8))
 (segment (start 116.007 64.453) (end 116.007 63.703) (width 0.25) (layer "F.Cu") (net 8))
 (segment (start 114.932 58.957) (end 114.932 60.222) (width 0.25) (layer "F.Cu") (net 8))
 (segment (start 113.097 58.317) (end 113.455 58.317) (width 0.25) (layer "F.Cu") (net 8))
 (segment (start 113.05 66.66) (end 113.46 66.25) (width 0.25) (layer "F.Cu") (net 8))
 (segment (start 116.007 61.297) (end 114.937 60.227) (width 0.25) (layer "F.Cu") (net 8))
 (segment (start 113.46 58.322) (end 114.606999 58.322) (width 0.25) (layer "F.Cu") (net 8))
 (segment (start 105.113299 53.3) (end 109.3 53.3) (width 0.25) (layer "F.Cu") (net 5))
 (segment (start 104.97 60.27) (end 104.325 60.915) (width 0.25) (layer "F.Cu") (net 5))
 (segment (start 109.3 53.3) (end 110.6 54.6) (width 0.25) (layer "F.Cu") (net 5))
 (segment (start 107.6 60.444) (end 107.592 60.452) (width 0.25) (layer "F.Cu") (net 5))
 (segment (start 104.97 60.27) (end 105.144 60.444) (width 0.25) (layer "F.Cu") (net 5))
 (segment (start 103.355 60.64928) (end 103.355 55.058299) (width 0.25) (layer "F.Cu") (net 5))
 (segment (start 104.325 60.915) (end 103.62072 60.915) (width 0.25) (layer "F.Cu") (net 5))
 (segment (start 103.62072 60.915) (end 103.355 60.64928) (width 0.25) (layer "F.Cu") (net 5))
 (segment (start 103.355 55.058299) (end 105.113299 53.3) (width 0.25) (layer "F.Cu") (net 5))
 (segment (start 105.144 60.444) (end 107.6 60.444) (width 0.25) (layer "F.Cu") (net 5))
 (segment (start 104.968 58.998) (end 104.97 59) (width 0.25) (layer "F.Cu") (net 1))
 (segment (start 106.686 59.03) (end 107.6 59.944) (width 0.25) (layer "F.Cu") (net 1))
 (segment (start 104.968 59) (end 104.968 58.998) (width 0.25) (layer "F.Cu") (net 1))
 (segment (start 106.686 59) (end 106.686 59.03) (width 0.25) (layer "F.Cu") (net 1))
 (segment (start 104.97 59) (end 104.968 59) (width 0.25) (layer "F.Cu") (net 1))
 (segment (start 104.97 58.93) (end 108.1 55.8) (width 0.25) (layer "F.Cu") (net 1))
 (segment (start 104.97 59) (end 106.686 59) (width 0.25) (layer "F.Cu") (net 1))
 (segment (start 104.97 59) (end 104.97 58.93) (width 0.25) (layer "F.Cu") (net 1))
 (segment (start 108.1 55.8) (end 108.1 54.6) (width 0.25) (layer "F.Cu") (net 1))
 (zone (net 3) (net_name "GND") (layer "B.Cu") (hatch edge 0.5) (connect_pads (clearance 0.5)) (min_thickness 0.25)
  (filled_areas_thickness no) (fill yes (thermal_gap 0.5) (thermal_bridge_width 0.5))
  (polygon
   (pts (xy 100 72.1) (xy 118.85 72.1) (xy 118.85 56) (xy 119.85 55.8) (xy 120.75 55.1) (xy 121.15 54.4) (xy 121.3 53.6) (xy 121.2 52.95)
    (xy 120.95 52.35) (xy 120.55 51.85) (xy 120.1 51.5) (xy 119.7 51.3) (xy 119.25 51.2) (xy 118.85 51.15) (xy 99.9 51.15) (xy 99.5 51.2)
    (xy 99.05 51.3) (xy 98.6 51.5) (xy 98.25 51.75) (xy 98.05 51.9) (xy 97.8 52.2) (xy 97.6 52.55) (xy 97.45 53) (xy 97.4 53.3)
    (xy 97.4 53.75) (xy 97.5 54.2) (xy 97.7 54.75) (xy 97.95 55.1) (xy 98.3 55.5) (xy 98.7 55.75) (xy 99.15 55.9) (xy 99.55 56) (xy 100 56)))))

